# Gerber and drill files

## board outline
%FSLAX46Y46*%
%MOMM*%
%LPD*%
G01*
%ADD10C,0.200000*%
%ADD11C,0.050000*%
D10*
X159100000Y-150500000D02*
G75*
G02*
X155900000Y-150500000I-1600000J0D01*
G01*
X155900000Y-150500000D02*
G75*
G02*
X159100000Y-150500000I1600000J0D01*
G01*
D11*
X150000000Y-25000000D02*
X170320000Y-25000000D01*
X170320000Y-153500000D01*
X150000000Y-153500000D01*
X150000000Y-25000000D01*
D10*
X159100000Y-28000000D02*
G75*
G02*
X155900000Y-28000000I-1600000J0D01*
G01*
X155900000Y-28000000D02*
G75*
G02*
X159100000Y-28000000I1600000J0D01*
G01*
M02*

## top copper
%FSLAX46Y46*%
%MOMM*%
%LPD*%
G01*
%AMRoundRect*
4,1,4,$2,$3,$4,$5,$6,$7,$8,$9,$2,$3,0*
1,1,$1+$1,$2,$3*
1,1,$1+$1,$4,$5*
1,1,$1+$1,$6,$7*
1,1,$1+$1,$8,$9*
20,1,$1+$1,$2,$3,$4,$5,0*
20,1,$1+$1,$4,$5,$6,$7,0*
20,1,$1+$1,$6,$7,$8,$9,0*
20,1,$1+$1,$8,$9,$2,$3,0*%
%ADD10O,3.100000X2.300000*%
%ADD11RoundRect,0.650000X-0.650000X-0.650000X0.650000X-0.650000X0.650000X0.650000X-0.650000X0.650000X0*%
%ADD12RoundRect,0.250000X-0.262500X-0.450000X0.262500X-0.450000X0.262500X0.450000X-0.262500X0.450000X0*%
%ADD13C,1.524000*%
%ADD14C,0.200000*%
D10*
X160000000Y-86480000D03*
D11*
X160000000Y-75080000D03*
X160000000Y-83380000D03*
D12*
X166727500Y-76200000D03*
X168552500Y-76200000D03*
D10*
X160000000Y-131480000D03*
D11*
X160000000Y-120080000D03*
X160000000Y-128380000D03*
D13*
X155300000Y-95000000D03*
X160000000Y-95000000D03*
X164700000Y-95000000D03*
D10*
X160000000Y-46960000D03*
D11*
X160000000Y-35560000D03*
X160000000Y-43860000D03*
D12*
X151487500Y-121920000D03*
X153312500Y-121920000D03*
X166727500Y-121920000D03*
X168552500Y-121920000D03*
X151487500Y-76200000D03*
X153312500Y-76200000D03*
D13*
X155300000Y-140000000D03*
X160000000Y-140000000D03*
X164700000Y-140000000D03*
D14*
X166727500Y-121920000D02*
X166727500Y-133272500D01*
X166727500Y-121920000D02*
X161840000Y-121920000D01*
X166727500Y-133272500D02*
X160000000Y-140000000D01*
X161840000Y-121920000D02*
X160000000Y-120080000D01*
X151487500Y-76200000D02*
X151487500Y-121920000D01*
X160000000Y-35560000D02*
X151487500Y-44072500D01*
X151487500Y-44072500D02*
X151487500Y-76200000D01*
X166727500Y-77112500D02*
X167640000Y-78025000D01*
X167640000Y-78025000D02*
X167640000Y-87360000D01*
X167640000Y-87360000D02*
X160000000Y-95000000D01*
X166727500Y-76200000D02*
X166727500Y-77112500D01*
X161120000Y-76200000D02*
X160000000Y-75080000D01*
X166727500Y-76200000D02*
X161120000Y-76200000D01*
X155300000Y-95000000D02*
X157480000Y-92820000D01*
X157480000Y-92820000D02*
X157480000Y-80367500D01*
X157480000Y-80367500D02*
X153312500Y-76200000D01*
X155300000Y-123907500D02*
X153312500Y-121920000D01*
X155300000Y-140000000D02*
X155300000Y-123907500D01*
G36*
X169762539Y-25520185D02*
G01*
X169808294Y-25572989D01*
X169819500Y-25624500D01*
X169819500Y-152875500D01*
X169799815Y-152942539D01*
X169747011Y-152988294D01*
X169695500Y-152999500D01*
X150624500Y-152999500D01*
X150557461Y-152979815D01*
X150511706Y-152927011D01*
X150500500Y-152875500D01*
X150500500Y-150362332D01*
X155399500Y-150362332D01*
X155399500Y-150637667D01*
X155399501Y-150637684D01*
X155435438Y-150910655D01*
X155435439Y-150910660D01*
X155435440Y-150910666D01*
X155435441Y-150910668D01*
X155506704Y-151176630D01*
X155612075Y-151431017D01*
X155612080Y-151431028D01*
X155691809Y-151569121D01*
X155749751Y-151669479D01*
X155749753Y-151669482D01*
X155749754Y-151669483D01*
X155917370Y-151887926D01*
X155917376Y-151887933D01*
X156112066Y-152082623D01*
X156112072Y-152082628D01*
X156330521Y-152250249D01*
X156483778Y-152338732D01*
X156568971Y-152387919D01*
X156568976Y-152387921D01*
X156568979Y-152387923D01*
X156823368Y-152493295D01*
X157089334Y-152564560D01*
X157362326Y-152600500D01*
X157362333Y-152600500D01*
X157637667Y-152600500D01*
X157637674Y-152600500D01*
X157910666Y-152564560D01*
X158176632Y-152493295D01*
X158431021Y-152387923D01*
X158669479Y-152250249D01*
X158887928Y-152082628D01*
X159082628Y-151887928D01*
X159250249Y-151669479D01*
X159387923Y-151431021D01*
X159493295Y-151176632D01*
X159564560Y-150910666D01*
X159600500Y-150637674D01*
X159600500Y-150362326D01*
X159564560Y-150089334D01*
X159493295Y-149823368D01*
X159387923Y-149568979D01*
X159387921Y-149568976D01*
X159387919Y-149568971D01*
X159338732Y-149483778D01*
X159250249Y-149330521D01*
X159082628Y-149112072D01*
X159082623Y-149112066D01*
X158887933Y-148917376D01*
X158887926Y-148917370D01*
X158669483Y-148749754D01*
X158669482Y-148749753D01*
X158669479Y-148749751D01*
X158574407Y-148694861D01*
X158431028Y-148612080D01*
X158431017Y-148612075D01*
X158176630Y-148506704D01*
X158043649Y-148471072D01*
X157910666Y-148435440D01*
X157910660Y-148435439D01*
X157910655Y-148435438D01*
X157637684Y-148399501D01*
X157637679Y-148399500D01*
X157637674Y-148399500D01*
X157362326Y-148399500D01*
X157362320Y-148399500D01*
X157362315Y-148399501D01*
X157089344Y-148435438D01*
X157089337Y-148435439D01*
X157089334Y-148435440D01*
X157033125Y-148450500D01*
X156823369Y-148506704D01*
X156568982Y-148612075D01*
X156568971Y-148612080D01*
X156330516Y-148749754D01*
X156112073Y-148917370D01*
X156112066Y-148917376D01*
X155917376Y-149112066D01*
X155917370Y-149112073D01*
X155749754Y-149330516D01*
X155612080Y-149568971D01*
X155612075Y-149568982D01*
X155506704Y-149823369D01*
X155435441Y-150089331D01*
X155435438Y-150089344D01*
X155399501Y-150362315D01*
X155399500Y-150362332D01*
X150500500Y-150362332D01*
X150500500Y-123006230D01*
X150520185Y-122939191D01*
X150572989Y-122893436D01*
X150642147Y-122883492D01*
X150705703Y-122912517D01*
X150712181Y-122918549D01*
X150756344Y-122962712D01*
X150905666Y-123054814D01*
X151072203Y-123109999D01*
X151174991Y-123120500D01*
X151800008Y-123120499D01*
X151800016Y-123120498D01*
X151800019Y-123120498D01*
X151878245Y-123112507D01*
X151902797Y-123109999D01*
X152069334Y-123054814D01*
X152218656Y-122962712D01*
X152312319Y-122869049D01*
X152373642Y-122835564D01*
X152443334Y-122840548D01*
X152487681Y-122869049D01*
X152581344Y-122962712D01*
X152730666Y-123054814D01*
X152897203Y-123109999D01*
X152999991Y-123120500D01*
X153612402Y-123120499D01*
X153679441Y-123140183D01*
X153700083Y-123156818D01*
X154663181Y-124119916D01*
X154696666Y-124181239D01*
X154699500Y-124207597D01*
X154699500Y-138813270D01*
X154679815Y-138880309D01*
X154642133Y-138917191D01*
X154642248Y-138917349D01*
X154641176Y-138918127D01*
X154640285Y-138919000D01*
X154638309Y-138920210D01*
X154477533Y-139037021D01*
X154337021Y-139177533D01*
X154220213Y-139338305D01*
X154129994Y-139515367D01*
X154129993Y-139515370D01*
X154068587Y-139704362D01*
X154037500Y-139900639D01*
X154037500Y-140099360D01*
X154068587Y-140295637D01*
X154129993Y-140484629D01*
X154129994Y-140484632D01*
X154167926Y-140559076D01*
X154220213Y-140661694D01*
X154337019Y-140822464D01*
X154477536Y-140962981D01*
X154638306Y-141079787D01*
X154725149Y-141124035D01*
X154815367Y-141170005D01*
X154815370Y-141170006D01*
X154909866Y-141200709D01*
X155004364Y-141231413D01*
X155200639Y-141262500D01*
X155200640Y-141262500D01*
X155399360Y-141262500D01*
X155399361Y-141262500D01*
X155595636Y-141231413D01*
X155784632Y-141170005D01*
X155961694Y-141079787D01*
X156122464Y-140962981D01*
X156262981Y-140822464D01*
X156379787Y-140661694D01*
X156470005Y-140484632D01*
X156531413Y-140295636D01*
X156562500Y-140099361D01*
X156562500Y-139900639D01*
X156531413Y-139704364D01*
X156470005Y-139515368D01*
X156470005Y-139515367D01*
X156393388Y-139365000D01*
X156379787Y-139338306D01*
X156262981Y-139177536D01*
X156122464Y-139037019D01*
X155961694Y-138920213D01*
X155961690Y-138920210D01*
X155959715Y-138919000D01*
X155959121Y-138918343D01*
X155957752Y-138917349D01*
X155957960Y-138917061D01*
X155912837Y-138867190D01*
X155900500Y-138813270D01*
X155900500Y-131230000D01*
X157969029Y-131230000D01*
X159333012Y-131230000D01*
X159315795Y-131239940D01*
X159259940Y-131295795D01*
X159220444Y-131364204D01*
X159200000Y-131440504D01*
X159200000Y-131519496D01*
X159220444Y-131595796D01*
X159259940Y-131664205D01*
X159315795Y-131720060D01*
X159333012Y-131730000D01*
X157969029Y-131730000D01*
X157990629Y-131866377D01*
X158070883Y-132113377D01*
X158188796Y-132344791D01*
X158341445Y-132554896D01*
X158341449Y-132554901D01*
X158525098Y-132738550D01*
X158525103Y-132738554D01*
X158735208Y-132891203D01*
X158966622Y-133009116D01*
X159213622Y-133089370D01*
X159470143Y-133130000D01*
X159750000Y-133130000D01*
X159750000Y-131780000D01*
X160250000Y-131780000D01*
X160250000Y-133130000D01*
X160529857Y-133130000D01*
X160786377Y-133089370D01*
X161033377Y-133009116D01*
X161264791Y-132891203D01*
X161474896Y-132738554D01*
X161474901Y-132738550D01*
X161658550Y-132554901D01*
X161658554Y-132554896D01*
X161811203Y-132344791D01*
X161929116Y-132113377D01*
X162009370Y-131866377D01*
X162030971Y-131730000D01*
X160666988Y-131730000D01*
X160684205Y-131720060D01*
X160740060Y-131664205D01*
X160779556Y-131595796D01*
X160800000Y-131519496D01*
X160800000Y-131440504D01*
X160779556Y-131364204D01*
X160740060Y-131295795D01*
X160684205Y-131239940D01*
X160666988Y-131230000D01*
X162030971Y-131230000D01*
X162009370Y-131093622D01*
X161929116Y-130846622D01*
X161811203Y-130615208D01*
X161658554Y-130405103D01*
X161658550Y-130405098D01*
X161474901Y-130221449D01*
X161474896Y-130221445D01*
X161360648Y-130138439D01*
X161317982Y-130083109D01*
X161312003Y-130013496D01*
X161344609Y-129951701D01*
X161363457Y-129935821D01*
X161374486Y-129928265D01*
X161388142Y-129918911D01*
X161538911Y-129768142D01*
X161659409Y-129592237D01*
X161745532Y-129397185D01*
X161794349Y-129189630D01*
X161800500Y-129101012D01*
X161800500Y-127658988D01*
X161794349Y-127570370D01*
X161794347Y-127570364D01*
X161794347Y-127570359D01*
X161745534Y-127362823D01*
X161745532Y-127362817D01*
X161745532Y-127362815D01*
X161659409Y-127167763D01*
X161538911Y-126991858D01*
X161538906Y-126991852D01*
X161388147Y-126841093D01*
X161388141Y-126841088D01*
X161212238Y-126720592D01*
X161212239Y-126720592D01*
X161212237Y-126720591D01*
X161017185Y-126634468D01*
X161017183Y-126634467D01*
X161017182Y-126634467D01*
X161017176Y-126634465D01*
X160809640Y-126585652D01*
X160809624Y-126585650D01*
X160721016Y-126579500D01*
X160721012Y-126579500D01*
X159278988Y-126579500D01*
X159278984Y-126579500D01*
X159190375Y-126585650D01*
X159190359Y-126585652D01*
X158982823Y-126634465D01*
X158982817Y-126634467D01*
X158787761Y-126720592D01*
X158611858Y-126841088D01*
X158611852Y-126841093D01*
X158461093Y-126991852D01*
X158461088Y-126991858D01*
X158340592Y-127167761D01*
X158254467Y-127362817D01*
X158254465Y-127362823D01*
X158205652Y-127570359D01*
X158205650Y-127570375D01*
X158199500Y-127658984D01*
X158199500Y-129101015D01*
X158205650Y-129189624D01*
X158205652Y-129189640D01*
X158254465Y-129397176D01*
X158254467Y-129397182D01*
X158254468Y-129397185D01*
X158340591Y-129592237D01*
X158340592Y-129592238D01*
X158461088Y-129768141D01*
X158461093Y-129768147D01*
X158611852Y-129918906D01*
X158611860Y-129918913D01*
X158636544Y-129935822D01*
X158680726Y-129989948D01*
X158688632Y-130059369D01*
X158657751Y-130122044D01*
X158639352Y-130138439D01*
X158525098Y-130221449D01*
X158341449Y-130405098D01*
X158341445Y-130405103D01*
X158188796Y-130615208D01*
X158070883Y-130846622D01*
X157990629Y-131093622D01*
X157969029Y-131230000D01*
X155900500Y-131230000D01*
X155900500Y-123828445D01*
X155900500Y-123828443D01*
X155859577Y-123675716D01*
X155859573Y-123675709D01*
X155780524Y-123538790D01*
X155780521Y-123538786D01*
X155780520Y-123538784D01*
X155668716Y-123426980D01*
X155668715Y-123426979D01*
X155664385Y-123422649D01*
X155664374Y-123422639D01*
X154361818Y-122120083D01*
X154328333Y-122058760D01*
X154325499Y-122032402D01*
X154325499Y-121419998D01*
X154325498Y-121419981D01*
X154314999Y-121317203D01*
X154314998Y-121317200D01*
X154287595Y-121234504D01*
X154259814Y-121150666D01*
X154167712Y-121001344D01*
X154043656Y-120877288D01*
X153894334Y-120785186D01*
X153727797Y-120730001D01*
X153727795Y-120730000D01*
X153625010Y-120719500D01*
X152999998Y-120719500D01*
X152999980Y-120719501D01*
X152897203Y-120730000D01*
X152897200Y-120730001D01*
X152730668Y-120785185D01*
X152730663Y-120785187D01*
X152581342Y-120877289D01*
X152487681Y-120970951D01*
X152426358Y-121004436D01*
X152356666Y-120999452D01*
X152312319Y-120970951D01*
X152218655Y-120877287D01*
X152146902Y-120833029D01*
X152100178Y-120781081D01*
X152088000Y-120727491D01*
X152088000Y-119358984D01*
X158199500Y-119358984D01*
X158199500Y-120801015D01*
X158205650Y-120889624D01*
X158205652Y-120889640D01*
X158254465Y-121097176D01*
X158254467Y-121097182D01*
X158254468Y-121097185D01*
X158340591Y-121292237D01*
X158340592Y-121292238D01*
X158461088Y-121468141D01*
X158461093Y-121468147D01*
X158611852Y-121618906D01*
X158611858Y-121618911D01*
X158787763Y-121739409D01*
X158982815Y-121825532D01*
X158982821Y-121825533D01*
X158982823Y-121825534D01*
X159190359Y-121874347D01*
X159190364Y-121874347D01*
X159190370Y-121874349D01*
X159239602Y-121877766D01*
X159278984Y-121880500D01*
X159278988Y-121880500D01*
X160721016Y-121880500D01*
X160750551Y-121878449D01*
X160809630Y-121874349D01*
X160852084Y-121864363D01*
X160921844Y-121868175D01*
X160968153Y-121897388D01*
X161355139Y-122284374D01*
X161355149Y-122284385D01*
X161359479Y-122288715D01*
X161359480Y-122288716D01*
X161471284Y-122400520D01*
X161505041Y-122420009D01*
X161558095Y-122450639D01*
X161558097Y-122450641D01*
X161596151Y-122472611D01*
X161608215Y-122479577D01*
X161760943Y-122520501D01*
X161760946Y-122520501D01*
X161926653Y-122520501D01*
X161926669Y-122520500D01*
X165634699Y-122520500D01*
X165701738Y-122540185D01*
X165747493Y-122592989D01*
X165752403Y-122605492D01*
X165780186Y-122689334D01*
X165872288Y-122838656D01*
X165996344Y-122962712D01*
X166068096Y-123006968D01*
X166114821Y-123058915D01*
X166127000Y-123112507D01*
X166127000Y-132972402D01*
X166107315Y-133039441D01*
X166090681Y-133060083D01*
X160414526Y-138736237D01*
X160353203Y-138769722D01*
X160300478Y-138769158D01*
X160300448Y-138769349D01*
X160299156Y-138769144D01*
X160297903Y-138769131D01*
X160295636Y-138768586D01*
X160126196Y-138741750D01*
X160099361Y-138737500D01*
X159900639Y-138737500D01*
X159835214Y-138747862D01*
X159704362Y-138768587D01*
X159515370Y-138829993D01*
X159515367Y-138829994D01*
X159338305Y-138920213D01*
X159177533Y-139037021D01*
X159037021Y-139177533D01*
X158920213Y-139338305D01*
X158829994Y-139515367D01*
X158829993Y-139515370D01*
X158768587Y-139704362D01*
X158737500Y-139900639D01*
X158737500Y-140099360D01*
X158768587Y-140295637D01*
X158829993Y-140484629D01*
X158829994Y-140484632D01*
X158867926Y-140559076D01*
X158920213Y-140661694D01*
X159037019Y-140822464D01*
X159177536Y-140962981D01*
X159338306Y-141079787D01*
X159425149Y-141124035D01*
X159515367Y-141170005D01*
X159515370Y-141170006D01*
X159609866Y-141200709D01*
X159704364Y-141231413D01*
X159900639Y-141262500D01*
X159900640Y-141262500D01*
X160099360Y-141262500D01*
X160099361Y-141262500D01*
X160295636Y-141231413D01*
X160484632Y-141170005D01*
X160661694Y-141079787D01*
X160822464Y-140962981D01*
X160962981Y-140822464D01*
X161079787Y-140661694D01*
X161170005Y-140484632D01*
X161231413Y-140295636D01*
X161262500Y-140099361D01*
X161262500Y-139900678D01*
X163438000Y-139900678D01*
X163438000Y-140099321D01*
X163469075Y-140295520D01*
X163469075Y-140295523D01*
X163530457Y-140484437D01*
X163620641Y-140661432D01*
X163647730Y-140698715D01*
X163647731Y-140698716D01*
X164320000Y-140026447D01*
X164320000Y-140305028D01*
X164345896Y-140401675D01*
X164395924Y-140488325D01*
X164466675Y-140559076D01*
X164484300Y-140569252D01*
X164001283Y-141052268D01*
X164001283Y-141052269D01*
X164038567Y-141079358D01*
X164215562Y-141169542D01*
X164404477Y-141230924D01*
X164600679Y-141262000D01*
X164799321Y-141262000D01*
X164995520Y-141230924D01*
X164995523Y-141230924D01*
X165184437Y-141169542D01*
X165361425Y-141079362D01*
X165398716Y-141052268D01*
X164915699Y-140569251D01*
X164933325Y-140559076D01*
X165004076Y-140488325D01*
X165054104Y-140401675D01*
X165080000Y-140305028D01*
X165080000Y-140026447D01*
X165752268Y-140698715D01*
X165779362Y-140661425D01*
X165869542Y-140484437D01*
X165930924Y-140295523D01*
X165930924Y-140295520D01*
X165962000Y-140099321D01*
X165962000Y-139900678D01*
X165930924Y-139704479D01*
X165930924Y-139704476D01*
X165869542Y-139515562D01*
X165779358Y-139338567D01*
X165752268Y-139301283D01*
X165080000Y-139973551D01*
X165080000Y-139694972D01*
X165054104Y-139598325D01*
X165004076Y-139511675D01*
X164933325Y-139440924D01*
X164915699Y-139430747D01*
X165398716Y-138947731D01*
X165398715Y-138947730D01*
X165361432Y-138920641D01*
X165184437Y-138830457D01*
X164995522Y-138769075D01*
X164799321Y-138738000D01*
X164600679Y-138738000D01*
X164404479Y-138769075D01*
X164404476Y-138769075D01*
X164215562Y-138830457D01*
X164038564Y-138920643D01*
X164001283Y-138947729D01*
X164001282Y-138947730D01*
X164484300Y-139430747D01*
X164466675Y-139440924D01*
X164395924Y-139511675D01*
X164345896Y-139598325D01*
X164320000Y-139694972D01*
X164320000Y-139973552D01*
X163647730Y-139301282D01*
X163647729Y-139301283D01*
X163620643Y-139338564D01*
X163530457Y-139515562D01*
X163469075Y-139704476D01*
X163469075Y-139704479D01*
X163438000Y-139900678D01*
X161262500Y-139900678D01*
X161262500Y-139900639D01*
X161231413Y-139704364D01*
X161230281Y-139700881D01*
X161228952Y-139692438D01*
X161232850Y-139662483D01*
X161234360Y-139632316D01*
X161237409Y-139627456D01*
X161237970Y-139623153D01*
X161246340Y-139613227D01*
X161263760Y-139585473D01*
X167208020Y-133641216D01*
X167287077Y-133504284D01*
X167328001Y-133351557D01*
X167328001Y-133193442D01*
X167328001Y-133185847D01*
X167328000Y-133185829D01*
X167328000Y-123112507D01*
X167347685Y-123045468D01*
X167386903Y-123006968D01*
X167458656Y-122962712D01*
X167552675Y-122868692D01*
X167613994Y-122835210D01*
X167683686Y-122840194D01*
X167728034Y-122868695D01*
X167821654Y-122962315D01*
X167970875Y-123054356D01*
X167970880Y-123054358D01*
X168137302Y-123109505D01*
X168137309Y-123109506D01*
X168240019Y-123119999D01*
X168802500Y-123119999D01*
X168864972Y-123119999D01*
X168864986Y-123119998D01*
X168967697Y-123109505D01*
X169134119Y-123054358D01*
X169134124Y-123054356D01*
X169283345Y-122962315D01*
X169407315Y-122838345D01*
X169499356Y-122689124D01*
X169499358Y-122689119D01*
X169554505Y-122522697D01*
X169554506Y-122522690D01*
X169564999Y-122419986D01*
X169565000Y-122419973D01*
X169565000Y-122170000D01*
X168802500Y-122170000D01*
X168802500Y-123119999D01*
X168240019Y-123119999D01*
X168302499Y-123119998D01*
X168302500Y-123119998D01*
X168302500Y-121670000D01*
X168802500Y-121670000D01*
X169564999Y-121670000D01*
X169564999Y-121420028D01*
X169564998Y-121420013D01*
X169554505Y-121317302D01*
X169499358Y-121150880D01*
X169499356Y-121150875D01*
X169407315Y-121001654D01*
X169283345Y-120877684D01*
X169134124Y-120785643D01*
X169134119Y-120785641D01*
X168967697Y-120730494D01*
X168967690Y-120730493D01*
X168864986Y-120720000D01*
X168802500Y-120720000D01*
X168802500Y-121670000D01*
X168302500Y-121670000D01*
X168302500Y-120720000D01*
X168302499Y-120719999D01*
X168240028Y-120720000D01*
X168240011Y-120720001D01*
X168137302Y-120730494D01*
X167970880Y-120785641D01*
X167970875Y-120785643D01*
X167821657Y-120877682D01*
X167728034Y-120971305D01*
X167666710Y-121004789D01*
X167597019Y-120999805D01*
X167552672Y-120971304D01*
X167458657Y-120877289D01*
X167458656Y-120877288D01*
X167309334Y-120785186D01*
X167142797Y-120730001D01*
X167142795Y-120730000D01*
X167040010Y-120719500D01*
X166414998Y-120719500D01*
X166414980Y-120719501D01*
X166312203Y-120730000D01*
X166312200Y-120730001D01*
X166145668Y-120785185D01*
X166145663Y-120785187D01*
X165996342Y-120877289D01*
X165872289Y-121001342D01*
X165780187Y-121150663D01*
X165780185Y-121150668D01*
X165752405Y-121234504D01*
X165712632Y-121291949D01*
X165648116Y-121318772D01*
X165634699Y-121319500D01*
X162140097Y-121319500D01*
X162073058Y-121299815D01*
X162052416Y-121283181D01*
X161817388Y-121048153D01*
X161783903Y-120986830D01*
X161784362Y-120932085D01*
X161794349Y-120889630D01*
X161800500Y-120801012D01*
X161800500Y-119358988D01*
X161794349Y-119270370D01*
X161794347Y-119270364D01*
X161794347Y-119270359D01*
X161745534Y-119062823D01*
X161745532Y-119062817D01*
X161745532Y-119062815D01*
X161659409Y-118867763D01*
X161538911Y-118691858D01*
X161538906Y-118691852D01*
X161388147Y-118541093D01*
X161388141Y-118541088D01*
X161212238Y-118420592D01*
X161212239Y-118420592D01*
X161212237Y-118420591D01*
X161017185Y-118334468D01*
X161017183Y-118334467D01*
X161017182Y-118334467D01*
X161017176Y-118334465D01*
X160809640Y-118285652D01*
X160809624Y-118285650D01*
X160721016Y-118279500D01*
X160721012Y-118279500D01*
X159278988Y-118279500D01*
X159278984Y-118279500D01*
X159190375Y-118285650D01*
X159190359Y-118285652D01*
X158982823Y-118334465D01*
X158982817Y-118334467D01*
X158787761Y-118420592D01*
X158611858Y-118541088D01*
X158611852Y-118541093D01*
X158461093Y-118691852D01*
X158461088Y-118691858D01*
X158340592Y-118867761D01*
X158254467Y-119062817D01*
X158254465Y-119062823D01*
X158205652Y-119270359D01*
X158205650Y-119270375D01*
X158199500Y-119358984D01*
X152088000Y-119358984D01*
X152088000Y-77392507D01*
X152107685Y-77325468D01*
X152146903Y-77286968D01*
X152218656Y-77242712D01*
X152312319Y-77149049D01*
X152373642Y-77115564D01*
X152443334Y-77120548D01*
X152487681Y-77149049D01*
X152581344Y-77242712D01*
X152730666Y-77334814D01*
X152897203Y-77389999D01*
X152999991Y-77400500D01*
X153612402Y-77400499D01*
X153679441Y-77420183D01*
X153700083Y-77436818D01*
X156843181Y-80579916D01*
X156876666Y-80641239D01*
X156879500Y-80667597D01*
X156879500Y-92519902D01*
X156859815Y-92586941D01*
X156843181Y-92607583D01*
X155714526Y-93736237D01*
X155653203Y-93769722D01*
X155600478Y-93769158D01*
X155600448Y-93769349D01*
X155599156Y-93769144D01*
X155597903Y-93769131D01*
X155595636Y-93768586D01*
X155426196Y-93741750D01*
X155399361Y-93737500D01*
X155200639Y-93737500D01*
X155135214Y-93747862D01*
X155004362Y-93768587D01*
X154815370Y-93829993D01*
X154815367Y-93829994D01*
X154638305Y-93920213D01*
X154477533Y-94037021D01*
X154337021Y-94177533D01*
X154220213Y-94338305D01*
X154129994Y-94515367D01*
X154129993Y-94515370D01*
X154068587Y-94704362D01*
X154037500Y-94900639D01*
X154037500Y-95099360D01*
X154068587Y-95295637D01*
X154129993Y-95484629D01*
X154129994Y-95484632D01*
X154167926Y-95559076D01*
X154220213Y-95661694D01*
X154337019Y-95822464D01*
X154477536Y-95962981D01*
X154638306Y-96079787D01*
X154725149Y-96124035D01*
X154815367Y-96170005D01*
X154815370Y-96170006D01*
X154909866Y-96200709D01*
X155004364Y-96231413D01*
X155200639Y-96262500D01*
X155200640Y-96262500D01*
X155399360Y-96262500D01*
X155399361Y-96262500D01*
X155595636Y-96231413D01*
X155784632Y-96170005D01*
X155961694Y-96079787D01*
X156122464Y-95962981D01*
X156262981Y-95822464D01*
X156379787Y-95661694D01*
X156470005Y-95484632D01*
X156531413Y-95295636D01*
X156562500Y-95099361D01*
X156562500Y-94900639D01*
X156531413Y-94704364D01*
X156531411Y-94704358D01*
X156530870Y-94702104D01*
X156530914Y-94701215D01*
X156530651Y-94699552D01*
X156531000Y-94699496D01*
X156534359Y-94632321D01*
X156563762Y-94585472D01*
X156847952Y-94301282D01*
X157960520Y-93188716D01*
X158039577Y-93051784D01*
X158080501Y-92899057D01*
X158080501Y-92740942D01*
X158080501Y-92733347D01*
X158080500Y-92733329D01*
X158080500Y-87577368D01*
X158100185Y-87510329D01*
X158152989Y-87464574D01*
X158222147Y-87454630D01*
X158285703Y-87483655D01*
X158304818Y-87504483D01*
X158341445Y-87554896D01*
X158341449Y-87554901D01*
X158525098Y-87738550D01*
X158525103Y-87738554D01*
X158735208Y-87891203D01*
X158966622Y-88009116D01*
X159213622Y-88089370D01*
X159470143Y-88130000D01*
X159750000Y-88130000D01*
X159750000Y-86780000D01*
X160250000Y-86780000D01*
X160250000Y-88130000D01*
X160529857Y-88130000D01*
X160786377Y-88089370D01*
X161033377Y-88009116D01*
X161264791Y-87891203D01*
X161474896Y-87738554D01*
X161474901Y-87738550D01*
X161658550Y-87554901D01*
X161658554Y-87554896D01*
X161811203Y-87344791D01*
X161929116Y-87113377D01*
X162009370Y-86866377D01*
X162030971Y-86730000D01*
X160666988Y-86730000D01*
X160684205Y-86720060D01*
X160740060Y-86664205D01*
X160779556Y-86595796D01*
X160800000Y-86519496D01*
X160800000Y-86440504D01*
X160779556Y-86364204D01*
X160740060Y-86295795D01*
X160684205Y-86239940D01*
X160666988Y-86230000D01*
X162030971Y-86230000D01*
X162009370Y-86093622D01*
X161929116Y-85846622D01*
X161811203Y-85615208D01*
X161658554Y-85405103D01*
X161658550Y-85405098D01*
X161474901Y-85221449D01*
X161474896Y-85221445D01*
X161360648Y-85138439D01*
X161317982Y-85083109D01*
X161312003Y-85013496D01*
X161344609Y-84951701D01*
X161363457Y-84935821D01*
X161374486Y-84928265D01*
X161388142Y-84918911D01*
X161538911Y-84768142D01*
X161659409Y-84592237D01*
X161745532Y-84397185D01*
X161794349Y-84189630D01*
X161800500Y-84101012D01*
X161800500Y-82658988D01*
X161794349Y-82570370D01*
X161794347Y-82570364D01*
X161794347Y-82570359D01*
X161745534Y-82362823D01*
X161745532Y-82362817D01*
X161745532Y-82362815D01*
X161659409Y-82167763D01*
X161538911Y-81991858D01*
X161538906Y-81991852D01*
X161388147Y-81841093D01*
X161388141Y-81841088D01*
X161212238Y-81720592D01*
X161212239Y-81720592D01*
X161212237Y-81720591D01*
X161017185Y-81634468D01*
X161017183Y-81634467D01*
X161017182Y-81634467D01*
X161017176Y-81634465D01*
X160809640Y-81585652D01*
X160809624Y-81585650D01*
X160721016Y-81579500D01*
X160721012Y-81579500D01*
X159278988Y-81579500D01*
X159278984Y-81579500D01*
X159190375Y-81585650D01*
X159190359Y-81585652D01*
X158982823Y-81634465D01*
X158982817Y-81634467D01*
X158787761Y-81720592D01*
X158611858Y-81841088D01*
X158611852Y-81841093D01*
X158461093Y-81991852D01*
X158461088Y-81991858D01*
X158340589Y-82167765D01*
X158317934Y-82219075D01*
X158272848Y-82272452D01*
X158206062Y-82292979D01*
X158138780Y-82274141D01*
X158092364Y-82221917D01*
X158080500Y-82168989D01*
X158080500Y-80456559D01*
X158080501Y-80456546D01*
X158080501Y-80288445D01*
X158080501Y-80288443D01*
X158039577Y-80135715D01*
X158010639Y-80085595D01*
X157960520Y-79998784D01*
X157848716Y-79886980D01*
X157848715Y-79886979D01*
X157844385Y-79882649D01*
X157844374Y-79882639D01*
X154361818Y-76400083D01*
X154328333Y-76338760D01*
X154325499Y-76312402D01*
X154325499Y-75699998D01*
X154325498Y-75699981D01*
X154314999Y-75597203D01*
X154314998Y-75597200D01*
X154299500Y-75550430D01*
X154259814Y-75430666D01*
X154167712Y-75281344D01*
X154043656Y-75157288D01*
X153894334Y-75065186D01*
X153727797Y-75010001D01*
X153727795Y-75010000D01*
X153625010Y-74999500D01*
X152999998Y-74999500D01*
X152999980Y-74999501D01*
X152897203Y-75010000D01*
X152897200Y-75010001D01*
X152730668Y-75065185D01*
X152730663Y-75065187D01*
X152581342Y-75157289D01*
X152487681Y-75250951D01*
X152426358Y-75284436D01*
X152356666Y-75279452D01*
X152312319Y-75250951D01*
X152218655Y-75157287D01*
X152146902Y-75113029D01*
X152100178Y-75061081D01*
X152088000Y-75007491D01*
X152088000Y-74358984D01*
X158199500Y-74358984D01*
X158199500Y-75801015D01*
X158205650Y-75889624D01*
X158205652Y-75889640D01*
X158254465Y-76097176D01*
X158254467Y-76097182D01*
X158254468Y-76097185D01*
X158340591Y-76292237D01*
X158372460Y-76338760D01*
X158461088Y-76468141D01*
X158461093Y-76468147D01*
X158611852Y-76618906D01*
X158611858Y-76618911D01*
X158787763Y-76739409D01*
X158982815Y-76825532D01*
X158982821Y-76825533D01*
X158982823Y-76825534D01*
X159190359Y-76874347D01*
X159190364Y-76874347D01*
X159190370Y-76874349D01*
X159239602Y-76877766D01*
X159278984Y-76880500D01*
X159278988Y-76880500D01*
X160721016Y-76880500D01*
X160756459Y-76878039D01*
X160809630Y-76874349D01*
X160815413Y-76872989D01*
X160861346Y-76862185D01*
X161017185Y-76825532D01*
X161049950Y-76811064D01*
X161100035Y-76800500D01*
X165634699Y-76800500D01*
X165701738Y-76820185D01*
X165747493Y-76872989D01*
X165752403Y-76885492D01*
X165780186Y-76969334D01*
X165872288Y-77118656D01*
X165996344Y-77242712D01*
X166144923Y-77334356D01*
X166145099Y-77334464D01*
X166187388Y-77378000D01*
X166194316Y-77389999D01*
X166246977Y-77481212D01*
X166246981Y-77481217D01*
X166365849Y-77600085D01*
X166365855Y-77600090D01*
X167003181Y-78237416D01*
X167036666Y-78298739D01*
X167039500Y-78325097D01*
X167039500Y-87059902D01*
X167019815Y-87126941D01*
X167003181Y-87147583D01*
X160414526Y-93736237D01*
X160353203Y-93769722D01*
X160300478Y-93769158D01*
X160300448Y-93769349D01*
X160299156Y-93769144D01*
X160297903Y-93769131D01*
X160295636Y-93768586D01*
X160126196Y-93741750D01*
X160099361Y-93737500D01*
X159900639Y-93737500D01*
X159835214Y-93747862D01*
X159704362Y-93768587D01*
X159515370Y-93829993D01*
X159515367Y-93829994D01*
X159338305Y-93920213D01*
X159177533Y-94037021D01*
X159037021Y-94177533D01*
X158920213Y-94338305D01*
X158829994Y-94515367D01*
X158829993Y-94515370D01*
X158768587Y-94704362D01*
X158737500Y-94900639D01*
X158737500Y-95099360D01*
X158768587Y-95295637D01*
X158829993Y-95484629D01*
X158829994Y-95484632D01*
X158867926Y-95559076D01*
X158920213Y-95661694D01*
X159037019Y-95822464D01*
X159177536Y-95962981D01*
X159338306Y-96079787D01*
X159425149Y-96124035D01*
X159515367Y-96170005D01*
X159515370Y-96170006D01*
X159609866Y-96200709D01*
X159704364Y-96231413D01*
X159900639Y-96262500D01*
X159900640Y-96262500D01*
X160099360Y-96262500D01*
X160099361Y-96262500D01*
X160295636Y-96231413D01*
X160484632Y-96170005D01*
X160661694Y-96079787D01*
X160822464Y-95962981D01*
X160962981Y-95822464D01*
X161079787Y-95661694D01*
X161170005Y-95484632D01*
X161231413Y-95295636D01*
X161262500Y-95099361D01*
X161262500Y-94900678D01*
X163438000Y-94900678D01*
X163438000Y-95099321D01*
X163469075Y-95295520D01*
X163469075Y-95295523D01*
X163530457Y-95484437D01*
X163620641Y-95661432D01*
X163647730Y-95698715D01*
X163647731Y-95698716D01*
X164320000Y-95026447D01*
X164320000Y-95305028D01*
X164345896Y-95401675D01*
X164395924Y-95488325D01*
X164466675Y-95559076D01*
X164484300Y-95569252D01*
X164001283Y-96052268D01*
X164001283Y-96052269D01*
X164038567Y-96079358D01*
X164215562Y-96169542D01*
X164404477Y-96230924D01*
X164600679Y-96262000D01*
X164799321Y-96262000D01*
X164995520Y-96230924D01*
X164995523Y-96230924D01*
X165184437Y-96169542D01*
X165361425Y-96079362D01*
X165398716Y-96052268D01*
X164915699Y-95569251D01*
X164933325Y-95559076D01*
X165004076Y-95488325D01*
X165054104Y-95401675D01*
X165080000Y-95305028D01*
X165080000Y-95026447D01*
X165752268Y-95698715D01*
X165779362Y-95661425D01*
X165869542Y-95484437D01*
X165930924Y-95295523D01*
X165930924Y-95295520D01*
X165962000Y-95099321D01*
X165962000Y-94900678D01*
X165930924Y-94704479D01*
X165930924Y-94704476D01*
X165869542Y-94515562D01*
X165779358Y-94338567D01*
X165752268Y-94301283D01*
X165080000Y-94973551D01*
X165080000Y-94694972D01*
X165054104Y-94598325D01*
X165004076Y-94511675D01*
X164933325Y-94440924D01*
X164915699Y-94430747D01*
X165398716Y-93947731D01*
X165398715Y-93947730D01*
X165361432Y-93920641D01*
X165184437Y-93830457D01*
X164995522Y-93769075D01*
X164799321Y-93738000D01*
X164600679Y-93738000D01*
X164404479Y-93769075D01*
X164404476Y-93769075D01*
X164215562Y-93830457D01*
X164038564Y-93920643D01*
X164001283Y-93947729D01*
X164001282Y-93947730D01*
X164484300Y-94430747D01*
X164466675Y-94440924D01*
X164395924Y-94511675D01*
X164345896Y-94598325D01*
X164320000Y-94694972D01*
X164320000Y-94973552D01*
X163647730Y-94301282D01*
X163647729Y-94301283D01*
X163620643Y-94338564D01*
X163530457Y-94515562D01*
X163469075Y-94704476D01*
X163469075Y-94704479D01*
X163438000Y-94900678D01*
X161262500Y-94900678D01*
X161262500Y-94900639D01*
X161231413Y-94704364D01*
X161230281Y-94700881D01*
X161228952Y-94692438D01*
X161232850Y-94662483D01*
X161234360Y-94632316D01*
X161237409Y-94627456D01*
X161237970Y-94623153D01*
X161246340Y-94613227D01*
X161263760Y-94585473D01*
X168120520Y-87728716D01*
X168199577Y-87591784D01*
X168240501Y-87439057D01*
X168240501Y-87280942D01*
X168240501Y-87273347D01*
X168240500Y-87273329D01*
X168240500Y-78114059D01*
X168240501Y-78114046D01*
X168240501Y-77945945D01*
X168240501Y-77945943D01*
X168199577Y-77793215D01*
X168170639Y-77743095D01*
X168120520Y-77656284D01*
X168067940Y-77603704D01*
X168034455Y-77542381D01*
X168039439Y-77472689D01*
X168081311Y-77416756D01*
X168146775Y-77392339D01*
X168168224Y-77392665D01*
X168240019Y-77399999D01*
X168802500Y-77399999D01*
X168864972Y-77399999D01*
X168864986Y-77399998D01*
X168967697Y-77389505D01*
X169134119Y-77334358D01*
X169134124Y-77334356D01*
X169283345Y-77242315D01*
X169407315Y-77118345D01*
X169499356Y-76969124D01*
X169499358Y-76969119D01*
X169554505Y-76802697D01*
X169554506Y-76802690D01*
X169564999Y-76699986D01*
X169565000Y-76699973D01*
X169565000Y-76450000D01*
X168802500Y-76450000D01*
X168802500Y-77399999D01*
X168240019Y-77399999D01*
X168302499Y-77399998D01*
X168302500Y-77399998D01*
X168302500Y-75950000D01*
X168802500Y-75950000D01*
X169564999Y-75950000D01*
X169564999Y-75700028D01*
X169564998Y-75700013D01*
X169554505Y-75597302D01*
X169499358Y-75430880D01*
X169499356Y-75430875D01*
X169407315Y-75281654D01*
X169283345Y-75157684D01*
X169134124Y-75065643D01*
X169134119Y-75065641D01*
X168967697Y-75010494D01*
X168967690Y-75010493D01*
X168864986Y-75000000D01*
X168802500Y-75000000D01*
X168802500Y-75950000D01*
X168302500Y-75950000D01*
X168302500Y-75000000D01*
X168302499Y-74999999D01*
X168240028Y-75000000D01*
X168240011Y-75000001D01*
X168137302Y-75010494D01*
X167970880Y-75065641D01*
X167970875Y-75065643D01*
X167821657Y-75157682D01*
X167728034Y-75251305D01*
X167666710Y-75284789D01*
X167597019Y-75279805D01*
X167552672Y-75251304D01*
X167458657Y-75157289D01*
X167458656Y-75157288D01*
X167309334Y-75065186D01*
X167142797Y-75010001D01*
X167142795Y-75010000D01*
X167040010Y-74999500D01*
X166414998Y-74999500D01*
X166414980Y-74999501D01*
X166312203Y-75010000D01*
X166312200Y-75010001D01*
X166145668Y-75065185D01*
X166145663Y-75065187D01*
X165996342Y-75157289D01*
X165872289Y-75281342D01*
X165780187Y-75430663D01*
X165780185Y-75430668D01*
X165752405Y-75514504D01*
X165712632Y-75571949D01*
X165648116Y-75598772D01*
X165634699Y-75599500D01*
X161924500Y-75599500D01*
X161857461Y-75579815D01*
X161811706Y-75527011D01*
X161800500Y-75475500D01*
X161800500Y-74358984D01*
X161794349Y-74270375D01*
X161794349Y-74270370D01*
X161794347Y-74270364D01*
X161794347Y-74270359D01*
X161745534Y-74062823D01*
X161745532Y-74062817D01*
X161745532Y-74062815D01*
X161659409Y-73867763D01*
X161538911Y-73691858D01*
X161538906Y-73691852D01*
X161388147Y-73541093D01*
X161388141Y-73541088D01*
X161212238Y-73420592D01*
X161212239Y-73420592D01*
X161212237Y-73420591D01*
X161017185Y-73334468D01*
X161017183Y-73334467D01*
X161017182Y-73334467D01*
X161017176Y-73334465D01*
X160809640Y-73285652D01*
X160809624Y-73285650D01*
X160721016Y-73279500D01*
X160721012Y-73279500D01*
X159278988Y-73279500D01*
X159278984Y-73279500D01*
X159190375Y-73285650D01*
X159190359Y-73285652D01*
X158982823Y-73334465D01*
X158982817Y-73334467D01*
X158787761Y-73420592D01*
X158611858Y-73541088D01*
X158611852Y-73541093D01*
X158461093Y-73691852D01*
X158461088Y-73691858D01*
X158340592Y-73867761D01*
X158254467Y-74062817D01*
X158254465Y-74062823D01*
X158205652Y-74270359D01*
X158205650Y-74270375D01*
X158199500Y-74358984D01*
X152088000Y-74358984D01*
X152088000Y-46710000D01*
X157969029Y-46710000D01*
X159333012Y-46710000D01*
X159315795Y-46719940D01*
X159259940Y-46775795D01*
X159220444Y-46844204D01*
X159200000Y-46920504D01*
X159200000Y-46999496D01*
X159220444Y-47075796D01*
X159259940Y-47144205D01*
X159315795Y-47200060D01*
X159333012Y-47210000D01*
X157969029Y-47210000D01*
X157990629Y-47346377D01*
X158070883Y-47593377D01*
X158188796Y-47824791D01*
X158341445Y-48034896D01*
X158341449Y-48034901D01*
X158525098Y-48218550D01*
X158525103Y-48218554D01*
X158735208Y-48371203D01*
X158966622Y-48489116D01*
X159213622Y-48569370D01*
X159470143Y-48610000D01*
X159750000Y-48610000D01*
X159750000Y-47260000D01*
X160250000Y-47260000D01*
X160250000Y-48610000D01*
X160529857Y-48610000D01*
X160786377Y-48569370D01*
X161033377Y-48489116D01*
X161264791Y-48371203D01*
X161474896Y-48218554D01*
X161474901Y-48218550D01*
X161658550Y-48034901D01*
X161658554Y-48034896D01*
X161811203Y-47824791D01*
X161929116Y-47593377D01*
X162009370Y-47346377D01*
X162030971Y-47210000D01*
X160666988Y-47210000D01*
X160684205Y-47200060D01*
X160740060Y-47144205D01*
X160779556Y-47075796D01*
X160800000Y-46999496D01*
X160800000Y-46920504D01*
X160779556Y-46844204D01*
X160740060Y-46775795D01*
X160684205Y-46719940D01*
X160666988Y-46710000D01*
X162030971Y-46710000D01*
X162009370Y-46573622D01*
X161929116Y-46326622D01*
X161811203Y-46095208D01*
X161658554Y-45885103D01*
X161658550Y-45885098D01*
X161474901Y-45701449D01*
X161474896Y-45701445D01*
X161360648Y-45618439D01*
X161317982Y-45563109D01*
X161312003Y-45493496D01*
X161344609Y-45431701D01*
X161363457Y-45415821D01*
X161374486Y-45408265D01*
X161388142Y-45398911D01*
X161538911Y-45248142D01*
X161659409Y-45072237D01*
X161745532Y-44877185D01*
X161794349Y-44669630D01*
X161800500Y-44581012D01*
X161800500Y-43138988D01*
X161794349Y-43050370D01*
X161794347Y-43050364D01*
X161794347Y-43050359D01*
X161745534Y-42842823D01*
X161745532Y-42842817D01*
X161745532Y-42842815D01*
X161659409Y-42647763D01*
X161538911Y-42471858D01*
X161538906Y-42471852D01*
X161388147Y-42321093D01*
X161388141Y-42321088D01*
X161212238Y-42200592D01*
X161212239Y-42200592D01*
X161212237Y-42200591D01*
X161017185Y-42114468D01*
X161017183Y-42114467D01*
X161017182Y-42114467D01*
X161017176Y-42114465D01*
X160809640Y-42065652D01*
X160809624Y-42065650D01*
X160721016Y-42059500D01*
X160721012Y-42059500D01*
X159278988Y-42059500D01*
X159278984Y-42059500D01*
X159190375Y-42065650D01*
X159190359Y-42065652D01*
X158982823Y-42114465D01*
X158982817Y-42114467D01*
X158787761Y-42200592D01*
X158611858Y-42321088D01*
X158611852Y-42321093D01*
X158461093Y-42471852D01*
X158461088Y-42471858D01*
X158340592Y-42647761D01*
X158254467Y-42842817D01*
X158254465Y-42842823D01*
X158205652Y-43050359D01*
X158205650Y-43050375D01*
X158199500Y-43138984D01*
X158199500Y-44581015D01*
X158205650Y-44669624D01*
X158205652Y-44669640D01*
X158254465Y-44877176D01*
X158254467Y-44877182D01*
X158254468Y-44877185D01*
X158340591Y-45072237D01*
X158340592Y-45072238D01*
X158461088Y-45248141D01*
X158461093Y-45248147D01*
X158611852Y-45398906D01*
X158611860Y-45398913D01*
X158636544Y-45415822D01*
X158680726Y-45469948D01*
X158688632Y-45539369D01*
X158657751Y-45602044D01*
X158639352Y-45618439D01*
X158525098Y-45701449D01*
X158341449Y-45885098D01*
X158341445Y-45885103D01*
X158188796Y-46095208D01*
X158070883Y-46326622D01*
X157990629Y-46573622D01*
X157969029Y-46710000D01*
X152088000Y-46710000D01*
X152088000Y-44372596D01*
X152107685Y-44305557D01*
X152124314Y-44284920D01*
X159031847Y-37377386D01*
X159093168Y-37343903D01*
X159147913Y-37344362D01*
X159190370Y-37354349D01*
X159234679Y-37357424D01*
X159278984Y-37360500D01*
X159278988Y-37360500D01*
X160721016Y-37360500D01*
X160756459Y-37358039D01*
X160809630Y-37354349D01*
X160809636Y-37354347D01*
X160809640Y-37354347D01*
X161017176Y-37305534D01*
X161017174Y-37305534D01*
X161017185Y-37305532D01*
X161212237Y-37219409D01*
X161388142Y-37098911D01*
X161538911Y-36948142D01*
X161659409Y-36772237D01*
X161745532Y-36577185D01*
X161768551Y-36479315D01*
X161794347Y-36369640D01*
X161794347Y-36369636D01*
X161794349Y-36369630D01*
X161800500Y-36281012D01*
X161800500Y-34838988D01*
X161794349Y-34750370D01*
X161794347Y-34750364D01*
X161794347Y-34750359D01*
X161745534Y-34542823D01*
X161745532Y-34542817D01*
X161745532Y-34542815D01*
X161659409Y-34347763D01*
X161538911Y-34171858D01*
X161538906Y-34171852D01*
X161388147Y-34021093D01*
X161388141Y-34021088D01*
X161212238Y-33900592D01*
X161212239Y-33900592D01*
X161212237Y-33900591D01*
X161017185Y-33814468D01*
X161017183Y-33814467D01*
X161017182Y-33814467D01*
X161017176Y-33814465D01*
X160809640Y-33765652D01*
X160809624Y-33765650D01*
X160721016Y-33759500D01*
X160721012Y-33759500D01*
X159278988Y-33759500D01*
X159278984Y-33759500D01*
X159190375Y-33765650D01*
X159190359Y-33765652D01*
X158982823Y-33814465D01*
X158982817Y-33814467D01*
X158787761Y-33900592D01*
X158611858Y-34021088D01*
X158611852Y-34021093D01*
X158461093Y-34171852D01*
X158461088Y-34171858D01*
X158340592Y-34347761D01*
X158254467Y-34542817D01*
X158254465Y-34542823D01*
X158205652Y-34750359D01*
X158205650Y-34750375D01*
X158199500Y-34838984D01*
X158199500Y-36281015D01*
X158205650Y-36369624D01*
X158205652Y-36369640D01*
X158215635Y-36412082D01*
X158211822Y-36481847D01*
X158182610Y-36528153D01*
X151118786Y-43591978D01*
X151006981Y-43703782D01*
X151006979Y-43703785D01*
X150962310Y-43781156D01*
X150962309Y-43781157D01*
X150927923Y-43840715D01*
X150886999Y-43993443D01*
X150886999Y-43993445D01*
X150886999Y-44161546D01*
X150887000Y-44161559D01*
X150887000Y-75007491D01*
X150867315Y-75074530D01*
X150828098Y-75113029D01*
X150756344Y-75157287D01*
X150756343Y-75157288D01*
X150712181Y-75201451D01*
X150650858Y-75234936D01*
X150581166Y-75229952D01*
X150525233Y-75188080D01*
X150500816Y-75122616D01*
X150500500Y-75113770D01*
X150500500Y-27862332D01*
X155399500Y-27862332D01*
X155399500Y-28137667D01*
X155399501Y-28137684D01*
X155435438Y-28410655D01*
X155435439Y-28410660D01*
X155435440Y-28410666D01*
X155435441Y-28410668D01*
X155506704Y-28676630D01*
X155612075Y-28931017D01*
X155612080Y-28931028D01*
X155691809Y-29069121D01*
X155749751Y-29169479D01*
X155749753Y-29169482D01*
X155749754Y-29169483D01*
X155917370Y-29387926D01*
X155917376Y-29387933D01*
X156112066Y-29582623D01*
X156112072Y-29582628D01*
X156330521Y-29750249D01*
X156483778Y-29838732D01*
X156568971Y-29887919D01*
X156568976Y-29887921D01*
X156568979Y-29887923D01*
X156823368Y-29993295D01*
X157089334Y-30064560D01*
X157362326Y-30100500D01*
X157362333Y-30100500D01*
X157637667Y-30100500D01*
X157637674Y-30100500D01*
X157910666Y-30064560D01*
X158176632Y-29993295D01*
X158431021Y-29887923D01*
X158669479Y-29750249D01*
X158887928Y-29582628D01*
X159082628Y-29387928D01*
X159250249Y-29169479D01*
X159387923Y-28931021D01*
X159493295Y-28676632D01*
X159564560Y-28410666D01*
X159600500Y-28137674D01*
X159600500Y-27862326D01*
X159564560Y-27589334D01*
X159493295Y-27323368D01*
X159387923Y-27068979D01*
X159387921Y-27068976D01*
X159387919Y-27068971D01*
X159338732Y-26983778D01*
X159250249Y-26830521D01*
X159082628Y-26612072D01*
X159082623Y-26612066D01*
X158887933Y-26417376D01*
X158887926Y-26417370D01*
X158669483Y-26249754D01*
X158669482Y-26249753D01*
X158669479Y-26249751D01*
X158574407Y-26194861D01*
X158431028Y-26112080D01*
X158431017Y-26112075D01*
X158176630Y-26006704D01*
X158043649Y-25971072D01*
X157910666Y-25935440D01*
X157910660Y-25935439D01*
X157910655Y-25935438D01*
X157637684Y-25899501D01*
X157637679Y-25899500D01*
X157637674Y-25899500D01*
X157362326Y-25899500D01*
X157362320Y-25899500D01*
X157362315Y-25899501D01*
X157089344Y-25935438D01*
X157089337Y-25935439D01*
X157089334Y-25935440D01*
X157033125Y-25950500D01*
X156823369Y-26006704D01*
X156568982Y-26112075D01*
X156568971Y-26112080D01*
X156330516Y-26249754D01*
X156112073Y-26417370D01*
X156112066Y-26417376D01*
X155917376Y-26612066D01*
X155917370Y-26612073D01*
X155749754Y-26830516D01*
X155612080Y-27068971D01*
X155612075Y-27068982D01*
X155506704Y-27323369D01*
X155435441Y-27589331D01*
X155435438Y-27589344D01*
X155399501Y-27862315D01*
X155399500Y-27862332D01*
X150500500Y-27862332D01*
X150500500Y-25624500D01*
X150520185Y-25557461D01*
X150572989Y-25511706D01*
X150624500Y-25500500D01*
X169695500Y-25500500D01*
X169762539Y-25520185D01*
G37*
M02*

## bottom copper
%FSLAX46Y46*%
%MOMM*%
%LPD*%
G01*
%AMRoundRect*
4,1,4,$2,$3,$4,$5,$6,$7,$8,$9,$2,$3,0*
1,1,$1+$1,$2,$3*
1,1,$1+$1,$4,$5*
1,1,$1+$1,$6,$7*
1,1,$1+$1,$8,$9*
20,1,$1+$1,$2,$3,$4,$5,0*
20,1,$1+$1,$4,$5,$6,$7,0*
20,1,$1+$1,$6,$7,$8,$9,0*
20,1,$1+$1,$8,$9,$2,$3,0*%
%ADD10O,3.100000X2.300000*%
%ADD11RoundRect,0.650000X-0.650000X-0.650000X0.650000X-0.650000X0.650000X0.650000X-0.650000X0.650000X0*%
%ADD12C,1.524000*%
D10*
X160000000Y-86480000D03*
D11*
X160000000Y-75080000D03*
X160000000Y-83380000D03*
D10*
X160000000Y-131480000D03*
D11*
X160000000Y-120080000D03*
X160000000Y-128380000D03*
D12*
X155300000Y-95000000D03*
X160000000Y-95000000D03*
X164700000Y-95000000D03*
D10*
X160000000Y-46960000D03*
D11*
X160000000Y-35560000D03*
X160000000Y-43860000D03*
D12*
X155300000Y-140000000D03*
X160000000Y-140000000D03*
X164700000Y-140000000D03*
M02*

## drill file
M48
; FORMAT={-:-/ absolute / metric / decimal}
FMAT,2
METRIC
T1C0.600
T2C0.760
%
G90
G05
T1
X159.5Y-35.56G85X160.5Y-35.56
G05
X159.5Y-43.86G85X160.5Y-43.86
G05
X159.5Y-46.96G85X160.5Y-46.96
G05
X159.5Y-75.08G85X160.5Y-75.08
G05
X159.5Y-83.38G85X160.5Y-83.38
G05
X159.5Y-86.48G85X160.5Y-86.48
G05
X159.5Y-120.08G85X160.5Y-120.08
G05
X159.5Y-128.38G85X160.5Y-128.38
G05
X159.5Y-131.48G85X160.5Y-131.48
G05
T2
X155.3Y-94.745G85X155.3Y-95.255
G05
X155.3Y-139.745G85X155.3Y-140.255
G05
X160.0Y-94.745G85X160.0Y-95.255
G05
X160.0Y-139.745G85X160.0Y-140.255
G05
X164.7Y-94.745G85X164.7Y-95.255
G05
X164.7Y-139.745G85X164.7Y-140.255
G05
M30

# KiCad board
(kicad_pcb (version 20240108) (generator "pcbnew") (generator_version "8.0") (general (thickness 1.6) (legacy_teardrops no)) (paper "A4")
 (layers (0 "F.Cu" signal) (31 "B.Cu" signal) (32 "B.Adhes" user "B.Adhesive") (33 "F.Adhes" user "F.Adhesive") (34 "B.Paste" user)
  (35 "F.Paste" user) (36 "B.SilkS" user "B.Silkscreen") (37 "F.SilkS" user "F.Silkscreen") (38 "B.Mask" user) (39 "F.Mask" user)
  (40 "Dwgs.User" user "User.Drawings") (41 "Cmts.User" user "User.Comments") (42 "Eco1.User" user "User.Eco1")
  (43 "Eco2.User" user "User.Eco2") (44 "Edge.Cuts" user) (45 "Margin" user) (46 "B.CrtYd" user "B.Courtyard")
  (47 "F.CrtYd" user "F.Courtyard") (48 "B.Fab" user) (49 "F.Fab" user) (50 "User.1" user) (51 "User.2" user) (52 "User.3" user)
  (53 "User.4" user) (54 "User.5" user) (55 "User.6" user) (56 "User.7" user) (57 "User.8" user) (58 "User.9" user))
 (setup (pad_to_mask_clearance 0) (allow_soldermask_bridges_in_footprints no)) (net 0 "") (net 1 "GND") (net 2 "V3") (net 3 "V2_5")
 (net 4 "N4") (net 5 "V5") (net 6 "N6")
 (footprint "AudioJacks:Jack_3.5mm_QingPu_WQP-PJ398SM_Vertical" (layer "F.Cu") (at 160 80)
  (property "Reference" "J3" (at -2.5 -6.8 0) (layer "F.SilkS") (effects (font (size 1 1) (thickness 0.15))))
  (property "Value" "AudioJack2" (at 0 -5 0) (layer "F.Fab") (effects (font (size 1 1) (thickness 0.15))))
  (pad "S" thru_hole oval (at 0 6.48) (size 3.1 2.3) (drill oval 1.6 0.6) (layers "*.Cu" "*.Mask") (remove_unused_layers no) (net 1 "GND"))
  (pad "T" thru_hole roundrect (at 0 -4.92) (size 2.6 2.6) (drill oval 1.6 0.6) (layers "*.Cu" "*.Mask") (remove_unused_layers no)
   (roundrect_rratio 0.25) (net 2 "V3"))
  (pad "TN" thru_hole roundrect (at 0 3.38) (size 2.6 2.6) (drill oval 1.6 0.6) (layers "*.Cu" "*.Mask") (remove_unused_layers no)
   (roundrect_rratio 0.25)))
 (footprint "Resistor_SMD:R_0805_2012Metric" (layer "F.Cu") (at 167.64 76.2)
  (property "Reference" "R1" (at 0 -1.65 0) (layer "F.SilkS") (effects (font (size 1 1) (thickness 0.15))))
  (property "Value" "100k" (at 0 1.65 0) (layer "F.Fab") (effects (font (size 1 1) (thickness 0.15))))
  (pad "1" smd roundrect (at -0.9125 0) (size 1.025 1.4) (layers "F.Cu" "F.Paste" "F.Mask") (roundrect_rratio 0.243902439) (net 2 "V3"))
  (pad "2" smd roundrect (at 0.9125 0) (size 1.025 1.4) (layers "F.Cu" "F.Paste" "F.Mask") (roundrect_rratio 0.243902439) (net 1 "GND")))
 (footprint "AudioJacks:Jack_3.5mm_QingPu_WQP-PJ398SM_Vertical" (layer "F.Cu") (at 160 125)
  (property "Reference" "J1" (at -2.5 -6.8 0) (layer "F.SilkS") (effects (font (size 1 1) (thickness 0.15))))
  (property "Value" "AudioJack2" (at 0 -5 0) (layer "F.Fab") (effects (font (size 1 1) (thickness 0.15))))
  (pad "S" thru_hole oval (at 0 6.48) (size 3.1 2.3) (drill oval 1.6 0.6) (layers "*.Cu" "*.Mask") (remove_unused_layers no) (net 1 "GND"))
  (pad "T" thru_hole roundrect (at 0 -4.92) (size 2.6 2.6) (drill oval 1.6 0.6) (layers "*.Cu" "*.Mask") (remove_unused_layers no)
   (roundrect_rratio 0.25) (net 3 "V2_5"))
  (pad "TN" thru_hole roundrect (at 0 3.38) (size 2.6 2.6) (drill oval 1.6 0.6) (layers "*.Cu" "*.Mask") (remove_unused_layers no)
   (roundrect_rratio 0.25)))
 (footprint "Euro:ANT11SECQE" (layer "F.Cu") (at 160 95)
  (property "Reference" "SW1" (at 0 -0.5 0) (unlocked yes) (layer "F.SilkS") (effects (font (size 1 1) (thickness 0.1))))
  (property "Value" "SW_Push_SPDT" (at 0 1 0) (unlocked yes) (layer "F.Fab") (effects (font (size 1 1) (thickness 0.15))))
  (pad "1" thru_hole circle (at -4.7 0) (size 1.524 1.524) (drill oval 0.76 1.27) (layers "*.Cu" "*.Mask") (remove_unused_layers no)
   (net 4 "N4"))
  (pad "2" thru_hole circle (at 0 0) (size 1.524 1.524) (drill oval 0.76 1.27) (layers "*.Cu" "*.Mask") (remove_unused_layers no)
   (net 2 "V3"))
  (pad "3" thru_hole circle (at 4.7 0) (size 1.524 1.524) (drill oval 0.76 1.27) (layers "*.Cu" "*.Mask") (remove_unused_layers no)
   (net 1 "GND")))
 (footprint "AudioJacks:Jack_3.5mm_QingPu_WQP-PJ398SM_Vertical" (layer "F.Cu") (at 160 40.48)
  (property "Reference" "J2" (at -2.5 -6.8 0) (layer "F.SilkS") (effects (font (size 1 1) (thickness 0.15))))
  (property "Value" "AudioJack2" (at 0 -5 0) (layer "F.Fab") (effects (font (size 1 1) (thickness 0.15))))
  (pad "S" thru_hole oval (at 0 6.48) (size 3.1 2.3) (drill oval 1.6 0.6) (layers "*.Cu" "*.Mask") (remove_unused_layers no) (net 1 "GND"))
  (pad "T" thru_hole roundrect (at 0 -4.92) (size 2.6 2.6) (drill oval 1.6 0.6) (layers "*.Cu" "*.Mask") (remove_unused_layers no)
   (roundrect_rratio 0.25) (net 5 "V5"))
  (pad "TN" thru_hole roundrect (at 0 3.38) (size 2.6 2.6) (drill oval 1.6 0.6) (layers "*.Cu" "*.Mask") (remove_unused_layers no)
   (roundrect_rratio 0.25)))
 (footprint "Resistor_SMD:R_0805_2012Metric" (layer "F.Cu") (at 152.4 121.92)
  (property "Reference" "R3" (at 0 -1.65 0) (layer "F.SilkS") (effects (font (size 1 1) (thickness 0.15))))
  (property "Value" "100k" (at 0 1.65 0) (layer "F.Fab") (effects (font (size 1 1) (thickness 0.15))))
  (pad "1" smd roundrect (at -0.9125 0) (size 1.025 1.4) (layers "F.Cu" "F.Paste" "F.Mask") (roundrect_rratio 0.243902439) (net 5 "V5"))
  (pad "2" smd roundrect (at 0.9125 0) (size 1.025 1.4) (layers "F.Cu" "F.Paste" "F.Mask") (roundrect_rratio 0.243902439) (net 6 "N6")))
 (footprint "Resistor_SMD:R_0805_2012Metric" (layer "F.Cu") (at 167.64 121.92)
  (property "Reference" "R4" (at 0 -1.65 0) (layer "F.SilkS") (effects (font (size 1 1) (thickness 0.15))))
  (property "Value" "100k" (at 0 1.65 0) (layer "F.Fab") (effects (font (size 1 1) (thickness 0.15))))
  (pad "1" smd roundrect (at -0.9125 0) (size 1.025 1.4) (layers "F.Cu" "F.Paste" "F.Mask") (roundrect_rratio 0.243902439) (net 3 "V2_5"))
  (pad "2" smd roundrect (at 0.9125 0) (size 1.025 1.4) (layers "F.Cu" "F.Paste" "F.Mask") (roundrect_rratio 0.243902439) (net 1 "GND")))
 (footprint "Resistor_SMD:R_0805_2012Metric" (layer "F.Cu") (at 152.4 76.2)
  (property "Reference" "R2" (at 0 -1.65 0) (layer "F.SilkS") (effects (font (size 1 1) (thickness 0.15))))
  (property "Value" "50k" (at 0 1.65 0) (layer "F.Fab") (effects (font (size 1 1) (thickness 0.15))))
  (pad "1" smd roundrect (at -0.9125 0) (size 1.025 1.4) (layers "F.Cu" "F.Paste" "F.Mask") (roundrect_rratio 0.243902439) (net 5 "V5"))
  (pad "2" smd roundrect (at 0.9125 0) (size 1.025 1.4) (layers "F.Cu" "F.Paste" "F.Mask") (roundrect_rratio 0.243902439) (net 4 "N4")))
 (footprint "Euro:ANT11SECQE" (layer "F.Cu") (at 160 140)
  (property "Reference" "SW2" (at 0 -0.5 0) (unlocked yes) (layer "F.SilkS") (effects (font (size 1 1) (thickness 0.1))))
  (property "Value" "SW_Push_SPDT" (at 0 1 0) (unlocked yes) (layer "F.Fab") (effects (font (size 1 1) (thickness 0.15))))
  (pad "1" thru_hole circle (at -4.7 0) (size 1.524 1.524) (drill oval 0.76 1.27) (layers "*.Cu" "*.Mask") (remove_unused_layers no)
   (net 6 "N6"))
  (pad "2" thru_hole circle (at 0 0) (size 1.524 1.524) (drill oval 0.76 1.27) (layers "*.Cu" "*.Mask") (remove_unused_layers no)
   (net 3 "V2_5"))
  (pad "3" thru_hole circle (at 4.7 0) (size 1.524 1.524) (drill oval 0.76 1.27) (layers "*.Cu" "*.Mask") (remove_unused_layers no)
   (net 1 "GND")))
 (gr_circle (center 157.5 150.5) (end 159.1 150.5) (stroke (width 0.2) (type default)) (fill none) (layer "Edge.Cuts"))
 (gr_rect (start 150 25) (end 170.32 153.5) (stroke (width 0.05) (type default)) (fill none) (layer "Edge.Cuts"))
 (gr_circle (center 157.5 28) (end 159.1 28) (stroke (width 0.2) (type default)) (fill none) (layer "Edge.Cuts"))
 (segment (start 166.7275 121.92) (end 166.7275 133.2725) (width 0.2) (layer "F.Cu") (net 3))
 (segment (start 166.7275 121.92) (end 161.84 121.92) (width 0.2) (layer "F.Cu") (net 3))
 (segment (start 166.7275 133.2725) (end 160 140) (width 0.2) (layer "F.Cu") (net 3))
 (segment (start 161.84 121.92) (end 160 120.08) (width 0.2) (layer "F.Cu") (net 3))
 (segment (start 151.4875 76.2) (end 151.4875 121.92) (width 0.2) (layer "F.Cu") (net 5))
 (segment (start 160 35.56) (end 151.4875 44.0725) (width 0.2) (layer "F.Cu") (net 5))
 (segment (start 151.4875 44.0725) (end 151.4875 76.2) (width 0.2) (layer "F.Cu") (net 5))
 (segment (start 166.7275 77.1125) (end 167.64 78.025) (width 0.2) (layer "F.Cu") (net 2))
 (segment (start 167.64 78.025) (end 167.64 87.36) (width 0.2) (layer "F.Cu") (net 2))
 (segment (start 167.64 87.36) (end 160 95) (width 0.2) (layer "F.Cu") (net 2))
 (segment (start 166.7275 76.2) (end 166.7275 77.1125) (width 0.2) (layer "F.Cu") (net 2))
 (segment (start 161.12 76.2) (end 160 75.08) (width 0.2) (layer "F.Cu") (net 2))
 (segment (start 166.7275 76.2) (end 161.12 76.2) (width 0.2) (layer "F.Cu") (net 2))
 (segment (start 155.3 95) (end 157.48 92.82) (width 0.2) (layer "F.Cu") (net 4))
 (segment (start 157.48 92.82) (end 157.48 80.3675) (width 0.2) (layer "F.Cu") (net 4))
 (segment (start 157.48 80.3675) (end 153.3125 76.2) (width 0.2) (layer "F.Cu") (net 4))
 (segment (start 155.3 123.9075) (end 153.3125 121.92) (width 0.2) (layer "F.Cu") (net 6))
 (segment (start 155.3 140) (end 155.3 123.9075) (width 0.2) (layer "F.Cu") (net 6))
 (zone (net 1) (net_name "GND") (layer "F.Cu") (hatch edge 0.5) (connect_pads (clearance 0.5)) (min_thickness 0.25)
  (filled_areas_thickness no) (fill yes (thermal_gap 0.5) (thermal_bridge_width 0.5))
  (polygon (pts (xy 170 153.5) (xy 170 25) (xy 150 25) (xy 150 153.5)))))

